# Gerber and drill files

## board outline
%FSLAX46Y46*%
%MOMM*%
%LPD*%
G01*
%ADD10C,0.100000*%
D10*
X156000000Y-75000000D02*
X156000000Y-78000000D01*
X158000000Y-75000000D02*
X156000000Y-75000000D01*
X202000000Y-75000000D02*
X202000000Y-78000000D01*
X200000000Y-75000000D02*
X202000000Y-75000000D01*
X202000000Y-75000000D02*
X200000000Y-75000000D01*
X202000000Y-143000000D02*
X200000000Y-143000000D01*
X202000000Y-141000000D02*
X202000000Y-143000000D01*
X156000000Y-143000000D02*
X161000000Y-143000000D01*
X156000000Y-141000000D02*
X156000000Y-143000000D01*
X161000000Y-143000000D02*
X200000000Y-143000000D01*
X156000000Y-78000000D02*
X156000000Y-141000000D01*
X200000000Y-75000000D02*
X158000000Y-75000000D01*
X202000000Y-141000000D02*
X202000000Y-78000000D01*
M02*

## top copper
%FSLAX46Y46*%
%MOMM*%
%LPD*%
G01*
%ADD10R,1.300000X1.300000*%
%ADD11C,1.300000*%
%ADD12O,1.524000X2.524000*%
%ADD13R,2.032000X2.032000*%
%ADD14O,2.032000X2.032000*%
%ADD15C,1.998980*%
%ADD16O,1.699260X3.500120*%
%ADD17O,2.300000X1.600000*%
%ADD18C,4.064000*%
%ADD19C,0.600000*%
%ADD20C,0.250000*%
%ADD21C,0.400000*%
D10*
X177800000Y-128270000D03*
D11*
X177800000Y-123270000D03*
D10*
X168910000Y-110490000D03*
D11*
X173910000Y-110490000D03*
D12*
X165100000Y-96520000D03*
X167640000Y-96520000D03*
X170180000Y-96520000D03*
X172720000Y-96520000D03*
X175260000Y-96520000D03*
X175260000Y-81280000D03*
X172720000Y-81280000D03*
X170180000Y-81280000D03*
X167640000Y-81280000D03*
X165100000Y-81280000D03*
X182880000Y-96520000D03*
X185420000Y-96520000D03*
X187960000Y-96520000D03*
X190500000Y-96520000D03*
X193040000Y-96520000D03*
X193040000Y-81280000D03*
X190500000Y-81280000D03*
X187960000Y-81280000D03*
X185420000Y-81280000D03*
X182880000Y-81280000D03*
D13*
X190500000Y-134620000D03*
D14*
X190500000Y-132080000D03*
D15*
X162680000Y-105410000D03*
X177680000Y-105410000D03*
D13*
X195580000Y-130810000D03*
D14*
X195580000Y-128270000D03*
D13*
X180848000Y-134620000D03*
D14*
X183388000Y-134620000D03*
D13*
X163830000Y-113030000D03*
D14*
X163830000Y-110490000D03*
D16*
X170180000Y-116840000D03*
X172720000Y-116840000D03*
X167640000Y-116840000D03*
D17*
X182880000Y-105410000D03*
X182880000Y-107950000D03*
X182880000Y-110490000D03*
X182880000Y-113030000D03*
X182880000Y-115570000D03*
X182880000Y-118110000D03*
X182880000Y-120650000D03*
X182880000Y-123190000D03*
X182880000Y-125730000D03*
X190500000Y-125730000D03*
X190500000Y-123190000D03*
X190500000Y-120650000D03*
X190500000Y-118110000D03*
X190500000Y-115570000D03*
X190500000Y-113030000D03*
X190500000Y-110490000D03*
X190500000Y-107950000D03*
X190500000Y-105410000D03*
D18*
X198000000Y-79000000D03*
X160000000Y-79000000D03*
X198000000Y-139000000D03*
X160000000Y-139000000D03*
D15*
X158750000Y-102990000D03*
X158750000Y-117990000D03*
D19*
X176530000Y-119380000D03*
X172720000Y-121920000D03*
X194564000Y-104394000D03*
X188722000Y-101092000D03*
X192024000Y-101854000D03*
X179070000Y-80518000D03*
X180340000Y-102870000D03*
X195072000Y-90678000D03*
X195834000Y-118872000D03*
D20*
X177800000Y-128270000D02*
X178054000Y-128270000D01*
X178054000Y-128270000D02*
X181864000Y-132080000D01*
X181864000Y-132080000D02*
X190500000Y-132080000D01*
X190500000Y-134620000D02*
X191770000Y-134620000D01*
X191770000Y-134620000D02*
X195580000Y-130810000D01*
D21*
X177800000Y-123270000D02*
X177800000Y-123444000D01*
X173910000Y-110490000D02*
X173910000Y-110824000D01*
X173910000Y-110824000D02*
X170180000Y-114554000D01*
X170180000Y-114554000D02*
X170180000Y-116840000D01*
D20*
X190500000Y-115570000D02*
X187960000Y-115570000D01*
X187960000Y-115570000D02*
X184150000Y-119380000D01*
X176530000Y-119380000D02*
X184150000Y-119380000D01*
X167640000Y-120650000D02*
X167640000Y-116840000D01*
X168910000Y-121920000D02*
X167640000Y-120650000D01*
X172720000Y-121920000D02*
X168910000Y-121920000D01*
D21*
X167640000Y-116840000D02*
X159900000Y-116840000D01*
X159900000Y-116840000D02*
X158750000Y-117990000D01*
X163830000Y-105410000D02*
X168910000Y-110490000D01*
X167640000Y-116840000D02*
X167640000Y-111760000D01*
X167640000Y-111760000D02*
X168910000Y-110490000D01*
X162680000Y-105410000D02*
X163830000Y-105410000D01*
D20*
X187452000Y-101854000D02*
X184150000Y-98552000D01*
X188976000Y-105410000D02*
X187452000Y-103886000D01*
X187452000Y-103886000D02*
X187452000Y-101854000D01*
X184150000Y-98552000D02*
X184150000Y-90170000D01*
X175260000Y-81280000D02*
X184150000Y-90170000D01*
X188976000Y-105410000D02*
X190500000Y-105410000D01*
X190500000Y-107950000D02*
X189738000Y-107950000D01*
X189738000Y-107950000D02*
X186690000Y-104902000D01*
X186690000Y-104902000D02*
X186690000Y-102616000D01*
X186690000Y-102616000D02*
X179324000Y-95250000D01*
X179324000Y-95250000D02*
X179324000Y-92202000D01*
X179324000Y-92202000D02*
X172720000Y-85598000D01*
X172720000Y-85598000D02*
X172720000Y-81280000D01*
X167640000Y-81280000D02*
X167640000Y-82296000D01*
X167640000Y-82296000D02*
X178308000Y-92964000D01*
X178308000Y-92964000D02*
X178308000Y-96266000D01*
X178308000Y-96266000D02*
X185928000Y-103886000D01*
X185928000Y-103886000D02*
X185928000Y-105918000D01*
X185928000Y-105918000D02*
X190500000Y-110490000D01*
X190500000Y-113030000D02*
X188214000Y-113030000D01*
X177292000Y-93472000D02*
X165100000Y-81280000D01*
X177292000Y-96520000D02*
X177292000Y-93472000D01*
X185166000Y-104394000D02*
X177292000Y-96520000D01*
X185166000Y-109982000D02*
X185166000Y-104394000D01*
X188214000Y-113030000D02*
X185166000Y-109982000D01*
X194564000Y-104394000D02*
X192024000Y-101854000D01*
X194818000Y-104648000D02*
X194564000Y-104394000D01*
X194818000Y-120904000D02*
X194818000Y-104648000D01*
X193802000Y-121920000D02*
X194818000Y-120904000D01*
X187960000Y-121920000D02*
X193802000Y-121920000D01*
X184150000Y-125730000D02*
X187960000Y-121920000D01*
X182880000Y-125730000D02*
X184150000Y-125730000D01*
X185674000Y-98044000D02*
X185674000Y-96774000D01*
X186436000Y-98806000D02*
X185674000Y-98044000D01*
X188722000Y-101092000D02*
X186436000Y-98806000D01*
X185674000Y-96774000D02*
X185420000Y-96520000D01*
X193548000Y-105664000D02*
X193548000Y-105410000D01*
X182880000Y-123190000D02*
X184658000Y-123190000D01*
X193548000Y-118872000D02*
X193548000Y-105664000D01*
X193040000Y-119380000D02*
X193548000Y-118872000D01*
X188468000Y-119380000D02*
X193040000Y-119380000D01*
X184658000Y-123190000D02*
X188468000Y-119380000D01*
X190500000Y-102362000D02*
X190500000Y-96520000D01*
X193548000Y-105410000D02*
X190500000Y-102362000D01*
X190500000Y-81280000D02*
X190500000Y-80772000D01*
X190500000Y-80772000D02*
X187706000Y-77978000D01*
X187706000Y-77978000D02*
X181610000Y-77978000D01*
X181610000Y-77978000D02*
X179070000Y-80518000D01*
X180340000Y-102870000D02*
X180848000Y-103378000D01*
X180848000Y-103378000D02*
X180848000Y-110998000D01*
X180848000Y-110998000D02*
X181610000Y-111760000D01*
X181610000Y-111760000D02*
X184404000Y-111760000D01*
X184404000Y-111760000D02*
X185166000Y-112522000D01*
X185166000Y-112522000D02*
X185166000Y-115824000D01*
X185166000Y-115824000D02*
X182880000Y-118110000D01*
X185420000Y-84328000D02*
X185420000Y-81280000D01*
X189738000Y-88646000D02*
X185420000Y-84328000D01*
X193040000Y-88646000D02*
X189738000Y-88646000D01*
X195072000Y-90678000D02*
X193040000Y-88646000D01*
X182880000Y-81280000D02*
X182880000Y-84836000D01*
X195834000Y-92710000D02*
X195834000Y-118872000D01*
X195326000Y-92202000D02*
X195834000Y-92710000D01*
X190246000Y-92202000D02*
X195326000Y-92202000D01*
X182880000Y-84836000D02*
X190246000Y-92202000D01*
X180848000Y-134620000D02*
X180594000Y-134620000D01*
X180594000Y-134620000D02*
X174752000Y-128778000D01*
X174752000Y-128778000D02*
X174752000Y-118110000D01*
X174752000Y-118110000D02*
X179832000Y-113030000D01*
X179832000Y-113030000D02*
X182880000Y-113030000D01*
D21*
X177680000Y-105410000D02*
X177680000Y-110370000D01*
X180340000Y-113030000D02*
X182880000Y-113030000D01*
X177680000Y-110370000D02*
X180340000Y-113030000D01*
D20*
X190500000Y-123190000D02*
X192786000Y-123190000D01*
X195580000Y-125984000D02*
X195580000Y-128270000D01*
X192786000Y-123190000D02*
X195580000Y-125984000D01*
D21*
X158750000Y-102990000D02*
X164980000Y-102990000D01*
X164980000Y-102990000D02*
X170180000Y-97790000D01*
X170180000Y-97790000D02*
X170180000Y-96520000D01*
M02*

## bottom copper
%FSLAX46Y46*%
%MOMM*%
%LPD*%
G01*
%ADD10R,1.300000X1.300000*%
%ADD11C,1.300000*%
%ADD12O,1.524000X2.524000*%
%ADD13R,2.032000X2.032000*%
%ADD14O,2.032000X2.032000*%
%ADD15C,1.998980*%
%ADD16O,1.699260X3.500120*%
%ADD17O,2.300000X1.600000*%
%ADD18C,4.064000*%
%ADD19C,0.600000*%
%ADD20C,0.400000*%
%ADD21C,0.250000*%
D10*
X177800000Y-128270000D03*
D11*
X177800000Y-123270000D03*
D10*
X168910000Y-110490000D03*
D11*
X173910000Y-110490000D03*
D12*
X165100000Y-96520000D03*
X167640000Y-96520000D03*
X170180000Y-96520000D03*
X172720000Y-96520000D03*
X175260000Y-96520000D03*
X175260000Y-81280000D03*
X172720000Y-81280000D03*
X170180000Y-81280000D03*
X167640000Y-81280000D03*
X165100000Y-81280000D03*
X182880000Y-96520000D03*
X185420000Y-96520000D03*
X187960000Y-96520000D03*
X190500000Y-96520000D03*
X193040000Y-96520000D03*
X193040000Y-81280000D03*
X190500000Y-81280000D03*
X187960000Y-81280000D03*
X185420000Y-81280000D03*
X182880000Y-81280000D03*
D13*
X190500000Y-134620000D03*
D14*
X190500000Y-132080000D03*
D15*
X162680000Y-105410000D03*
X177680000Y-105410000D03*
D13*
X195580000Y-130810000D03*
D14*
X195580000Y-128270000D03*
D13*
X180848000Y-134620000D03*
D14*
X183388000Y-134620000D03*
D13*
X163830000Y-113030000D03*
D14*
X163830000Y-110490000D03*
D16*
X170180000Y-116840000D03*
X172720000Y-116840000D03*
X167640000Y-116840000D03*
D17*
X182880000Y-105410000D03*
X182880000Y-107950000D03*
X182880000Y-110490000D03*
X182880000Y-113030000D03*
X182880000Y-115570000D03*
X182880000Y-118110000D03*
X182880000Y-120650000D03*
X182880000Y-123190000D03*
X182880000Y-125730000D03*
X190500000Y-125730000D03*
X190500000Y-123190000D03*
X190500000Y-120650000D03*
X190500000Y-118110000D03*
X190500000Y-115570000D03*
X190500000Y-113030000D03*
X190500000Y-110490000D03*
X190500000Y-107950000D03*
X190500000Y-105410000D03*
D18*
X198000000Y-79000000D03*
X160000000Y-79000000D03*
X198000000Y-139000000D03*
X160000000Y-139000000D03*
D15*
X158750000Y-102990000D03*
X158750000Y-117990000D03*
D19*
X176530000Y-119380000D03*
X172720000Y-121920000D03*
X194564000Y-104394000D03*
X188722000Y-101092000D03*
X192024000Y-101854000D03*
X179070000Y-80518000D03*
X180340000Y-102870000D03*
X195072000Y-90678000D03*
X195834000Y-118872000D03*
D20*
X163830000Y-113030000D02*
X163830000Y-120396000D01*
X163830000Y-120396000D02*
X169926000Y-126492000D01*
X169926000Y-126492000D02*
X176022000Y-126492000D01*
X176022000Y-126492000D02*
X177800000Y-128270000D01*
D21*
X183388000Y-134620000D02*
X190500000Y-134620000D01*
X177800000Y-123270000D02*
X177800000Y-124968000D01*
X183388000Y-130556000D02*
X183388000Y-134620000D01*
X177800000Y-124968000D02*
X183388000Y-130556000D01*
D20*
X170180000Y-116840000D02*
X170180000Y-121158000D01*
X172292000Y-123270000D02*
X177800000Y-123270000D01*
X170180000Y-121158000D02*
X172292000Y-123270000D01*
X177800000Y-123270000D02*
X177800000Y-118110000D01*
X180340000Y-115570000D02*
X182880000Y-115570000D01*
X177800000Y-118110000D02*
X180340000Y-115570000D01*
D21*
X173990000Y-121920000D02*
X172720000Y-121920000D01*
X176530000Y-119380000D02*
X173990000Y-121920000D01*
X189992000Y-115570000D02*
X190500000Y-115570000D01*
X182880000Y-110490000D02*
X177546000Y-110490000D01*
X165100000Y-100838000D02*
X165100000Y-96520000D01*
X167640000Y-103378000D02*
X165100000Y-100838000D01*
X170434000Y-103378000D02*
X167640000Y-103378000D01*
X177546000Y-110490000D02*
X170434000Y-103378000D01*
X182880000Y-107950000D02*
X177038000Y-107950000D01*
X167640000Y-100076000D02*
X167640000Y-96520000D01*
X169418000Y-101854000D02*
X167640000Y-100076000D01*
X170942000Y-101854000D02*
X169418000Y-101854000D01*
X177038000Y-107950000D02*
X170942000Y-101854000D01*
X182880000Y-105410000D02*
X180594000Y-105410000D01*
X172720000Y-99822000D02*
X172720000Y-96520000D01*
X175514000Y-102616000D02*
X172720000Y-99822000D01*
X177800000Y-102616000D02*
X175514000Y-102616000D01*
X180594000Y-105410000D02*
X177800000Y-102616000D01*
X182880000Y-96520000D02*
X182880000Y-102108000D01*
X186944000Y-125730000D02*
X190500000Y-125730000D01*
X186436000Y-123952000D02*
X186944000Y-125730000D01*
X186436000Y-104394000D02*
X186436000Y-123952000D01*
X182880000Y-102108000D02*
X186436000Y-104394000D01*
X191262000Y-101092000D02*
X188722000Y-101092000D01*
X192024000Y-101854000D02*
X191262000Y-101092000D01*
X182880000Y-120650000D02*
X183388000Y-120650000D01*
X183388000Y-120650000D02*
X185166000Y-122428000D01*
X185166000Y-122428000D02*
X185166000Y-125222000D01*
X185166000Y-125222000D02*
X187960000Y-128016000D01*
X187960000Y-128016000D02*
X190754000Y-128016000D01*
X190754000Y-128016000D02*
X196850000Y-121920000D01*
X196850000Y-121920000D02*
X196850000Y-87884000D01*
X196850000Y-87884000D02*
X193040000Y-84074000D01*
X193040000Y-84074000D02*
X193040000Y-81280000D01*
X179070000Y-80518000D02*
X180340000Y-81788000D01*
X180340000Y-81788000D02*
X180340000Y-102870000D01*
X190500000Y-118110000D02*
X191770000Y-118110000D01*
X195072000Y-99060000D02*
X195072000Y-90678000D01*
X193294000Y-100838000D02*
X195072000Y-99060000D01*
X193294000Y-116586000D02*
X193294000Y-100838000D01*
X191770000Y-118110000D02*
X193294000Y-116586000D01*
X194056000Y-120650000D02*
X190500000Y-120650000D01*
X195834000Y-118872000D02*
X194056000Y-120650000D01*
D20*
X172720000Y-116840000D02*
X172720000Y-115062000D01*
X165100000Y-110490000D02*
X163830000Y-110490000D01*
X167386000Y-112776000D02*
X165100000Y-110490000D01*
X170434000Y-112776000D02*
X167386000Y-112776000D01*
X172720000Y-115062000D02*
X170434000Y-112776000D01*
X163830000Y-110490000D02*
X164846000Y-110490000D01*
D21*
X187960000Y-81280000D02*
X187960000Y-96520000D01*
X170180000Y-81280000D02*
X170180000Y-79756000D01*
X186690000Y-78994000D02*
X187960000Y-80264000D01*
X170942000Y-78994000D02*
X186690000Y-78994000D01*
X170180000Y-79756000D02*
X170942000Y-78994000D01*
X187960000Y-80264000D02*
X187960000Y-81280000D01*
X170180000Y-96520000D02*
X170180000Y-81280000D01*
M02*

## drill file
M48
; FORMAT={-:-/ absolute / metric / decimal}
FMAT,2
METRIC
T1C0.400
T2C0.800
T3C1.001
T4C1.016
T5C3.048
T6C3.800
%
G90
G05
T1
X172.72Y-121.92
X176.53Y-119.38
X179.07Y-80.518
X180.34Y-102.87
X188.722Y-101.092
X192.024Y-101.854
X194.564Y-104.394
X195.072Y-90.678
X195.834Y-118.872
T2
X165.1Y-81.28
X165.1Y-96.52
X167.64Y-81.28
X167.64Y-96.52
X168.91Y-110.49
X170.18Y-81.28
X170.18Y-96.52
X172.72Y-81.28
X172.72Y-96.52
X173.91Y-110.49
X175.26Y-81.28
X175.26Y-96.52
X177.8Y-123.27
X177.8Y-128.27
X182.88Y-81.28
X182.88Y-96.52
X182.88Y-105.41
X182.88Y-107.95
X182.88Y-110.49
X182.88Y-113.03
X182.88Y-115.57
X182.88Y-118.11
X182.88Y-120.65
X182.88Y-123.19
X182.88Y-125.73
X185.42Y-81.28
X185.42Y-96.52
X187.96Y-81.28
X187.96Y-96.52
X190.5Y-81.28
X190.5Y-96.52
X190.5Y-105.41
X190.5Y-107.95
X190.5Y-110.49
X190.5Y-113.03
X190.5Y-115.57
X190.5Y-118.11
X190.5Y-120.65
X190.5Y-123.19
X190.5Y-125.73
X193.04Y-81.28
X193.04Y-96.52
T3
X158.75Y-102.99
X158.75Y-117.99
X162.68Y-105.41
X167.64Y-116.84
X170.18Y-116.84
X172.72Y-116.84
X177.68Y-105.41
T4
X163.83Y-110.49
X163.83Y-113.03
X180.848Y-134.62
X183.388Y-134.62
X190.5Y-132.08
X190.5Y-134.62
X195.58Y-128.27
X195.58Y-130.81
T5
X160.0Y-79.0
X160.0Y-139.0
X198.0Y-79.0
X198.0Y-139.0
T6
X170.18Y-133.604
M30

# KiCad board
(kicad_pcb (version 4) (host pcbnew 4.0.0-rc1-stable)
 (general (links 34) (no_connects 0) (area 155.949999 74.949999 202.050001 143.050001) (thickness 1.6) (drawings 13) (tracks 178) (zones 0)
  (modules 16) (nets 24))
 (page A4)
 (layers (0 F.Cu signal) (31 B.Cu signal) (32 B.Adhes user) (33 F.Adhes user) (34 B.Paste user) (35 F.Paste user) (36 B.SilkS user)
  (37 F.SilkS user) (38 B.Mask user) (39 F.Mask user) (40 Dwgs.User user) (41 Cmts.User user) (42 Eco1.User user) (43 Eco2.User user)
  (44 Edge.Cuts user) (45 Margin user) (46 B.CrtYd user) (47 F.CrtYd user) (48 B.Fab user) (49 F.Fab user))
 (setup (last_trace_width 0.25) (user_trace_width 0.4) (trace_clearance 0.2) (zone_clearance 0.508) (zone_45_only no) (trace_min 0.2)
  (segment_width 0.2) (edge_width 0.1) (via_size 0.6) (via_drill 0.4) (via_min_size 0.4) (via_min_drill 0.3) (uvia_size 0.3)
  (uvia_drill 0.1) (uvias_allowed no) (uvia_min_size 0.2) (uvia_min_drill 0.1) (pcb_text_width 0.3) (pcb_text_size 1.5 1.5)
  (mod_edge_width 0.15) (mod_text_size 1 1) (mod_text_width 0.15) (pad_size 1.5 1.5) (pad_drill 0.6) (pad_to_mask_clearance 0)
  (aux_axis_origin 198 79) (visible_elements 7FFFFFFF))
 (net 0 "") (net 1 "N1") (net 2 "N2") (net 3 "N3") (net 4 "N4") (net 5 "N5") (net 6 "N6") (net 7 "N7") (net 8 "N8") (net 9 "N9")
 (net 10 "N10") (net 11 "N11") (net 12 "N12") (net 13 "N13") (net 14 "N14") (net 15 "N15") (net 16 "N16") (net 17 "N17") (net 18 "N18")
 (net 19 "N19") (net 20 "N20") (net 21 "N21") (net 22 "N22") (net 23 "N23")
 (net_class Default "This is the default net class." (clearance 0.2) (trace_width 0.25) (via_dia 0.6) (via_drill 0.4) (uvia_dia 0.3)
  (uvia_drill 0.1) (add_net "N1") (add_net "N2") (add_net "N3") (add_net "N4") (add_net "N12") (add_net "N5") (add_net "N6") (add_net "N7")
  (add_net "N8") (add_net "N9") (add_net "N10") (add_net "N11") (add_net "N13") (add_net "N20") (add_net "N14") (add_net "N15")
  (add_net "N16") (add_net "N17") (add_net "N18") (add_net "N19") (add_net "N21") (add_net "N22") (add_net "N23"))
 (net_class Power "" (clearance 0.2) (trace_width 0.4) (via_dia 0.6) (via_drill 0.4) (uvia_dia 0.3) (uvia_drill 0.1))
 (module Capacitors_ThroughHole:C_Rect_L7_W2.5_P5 (layer F.Cu) (at 177.8 128.27 90)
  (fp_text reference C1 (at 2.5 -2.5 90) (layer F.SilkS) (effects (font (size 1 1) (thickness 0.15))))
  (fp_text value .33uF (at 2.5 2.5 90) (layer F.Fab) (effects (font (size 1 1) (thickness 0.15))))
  (pad 1 thru_hole rect (at 0 0 90) (size 1.3 1.3) (drill 0.8) (layers *.Cu *.Mask F.SilkS) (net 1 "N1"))
  (pad 2 thru_hole circle (at 5 0 90) (size 1.3 1.3) (drill 0.8) (layers *.Cu *.Mask F.SilkS) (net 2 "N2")))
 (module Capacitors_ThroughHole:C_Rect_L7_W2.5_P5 (layer F.Cu) (at 168.91 110.49)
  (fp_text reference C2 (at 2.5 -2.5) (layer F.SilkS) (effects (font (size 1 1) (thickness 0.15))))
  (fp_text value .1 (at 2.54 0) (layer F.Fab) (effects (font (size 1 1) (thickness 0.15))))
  (pad 1 thru_hole rect (at 0 0) (size 1.3 1.3) (drill 0.8) (layers *.Cu *.Mask F.SilkS) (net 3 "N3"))
  (pad 2 thru_hole circle (at 5 0) (size 1.3 1.3) (drill 0.8) (layers *.Cu *.Mask F.SilkS) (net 2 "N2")))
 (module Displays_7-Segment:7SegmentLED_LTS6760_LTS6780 (layer F.Cu) (at 170.18 88.9)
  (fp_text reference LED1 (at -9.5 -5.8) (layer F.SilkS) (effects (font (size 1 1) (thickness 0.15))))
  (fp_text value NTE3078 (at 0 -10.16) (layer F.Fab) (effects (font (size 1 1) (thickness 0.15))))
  (pad 1 thru_hole oval (at -5.08 7.62) (size 1.524 2.524) (drill 0.8) (layers *.Cu *.Mask F.SilkS) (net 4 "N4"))
  (pad 2 thru_hole oval (at -2.54 7.62) (size 1.524 2.524) (drill 0.8) (layers *.Cu *.Mask F.SilkS) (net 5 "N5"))
  (pad 3 thru_hole oval (at 0 7.62) (size 1.524 2.524) (drill 0.8) (layers *.Cu *.Mask F.SilkS) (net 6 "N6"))
  (pad 4 thru_hole oval (at 2.54 7.62) (size 1.524 2.524) (drill 0.8) (layers *.Cu *.Mask F.SilkS) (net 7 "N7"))
  (pad 5 thru_hole oval (at 5.08 7.62) (size 1.524 2.524) (drill 0.8) (layers *.Cu *.Mask F.SilkS) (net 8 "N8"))
  (pad 6 thru_hole oval (at 5.08 -7.62) (size 1.524 2.524) (drill 0.8) (layers *.Cu *.Mask F.SilkS) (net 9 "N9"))
  (pad 7 thru_hole oval (at 2.54 -7.62) (size 1.524 2.524) (drill 0.8) (layers *.Cu *.Mask F.SilkS) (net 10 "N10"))
  (pad 8 thru_hole oval (at 0 -7.62) (size 1.524 2.524) (drill 0.8) (layers *.Cu *.Mask F.SilkS) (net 6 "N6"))
  (pad 9 thru_hole oval (at -2.54 -7.62) (size 1.524 2.524) (drill 0.8) (layers *.Cu *.Mask F.SilkS) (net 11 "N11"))
  (pad 10 thru_hole oval (at -5.08 -7.62) (size 1.524 2.524) (drill 0.8) (layers *.Cu *.Mask F.SilkS) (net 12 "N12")))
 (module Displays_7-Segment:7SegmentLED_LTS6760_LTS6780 (layer F.Cu) (at 187.96 88.9)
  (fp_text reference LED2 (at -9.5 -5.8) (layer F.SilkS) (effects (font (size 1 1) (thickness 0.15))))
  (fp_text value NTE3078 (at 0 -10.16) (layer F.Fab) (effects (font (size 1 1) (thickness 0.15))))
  (pad 1 thru_hole oval (at -5.08 7.62) (size 1.524 2.524) (drill 0.8) (layers *.Cu *.Mask F.SilkS) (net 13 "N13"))
  (pad 2 thru_hole oval (at -2.54 7.62) (size 1.524 2.524) (drill 0.8) (layers *.Cu *.Mask F.SilkS) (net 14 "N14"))
  (pad 3 thru_hole oval (at 0 7.62) (size 1.524 2.524) (drill 0.8) (layers *.Cu *.Mask F.SilkS) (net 6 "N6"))
  (pad 4 thru_hole oval (at 2.54 7.62) (size 1.524 2.524) (drill 0.8) (layers *.Cu *.Mask F.SilkS) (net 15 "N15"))
  (pad 5 thru_hole oval (at 5.08 7.62) (size 1.524 2.524) (drill 0.8) (layers *.Cu *.Mask F.SilkS) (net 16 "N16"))
  (pad 6 thru_hole oval (at 5.08 -7.62) (size 1.524 2.524) (drill 0.8) (layers *.Cu *.Mask F.SilkS) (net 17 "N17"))
  (pad 7 thru_hole oval (at 2.54 -7.62) (size 1.524 2.524) (drill 0.8) (layers *.Cu *.Mask F.SilkS) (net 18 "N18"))
  (pad 8 thru_hole oval (at 0 -7.62) (size 1.524 2.524) (drill 0.8) (layers *.Cu *.Mask F.SilkS) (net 6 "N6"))
  (pad 9 thru_hole oval (at -2.54 -7.62) (size 1.524 2.524) (drill 0.8) (layers *.Cu *.Mask F.SilkS) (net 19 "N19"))
  (pad 10 thru_hole oval (at -5.08 -7.62) (size 1.524 2.524) (drill 0.8) (layers *.Cu *.Mask F.SilkS) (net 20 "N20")))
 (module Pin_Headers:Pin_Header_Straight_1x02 (layer F.Cu) (at 190.5 134.62 180)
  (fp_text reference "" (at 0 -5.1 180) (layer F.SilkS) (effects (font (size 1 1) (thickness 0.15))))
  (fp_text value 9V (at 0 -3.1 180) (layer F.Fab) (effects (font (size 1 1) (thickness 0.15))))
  (pad 1 thru_hole rect (at 0 0 180) (size 2.032 2.032) (drill 1.016) (layers *.Cu *.Mask F.SilkS) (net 2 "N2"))
  (pad 2 thru_hole oval (at 0 2.54 180) (size 2.032 2.032) (drill 1.016) (layers *.Cu *.Mask F.SilkS) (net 1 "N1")))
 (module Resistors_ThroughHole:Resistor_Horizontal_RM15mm (layer F.Cu) (at 170.18 105.41)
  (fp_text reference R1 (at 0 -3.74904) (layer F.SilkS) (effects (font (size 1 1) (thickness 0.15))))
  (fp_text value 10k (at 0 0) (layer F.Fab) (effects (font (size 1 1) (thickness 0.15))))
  (pad 1 thru_hole circle (at -7.5 0) (size 1.99898 1.99898) (drill 1.00076) (layers *.Cu *.SilkS *.Mask) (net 3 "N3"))
  (pad 2 thru_hole circle (at 7.5 0) (size 1.99898 1.99898) (drill 1.00076) (layers *.Cu *.SilkS *.Mask) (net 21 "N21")))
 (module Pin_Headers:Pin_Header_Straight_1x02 (layer F.Cu) (at 195.58 130.81 180)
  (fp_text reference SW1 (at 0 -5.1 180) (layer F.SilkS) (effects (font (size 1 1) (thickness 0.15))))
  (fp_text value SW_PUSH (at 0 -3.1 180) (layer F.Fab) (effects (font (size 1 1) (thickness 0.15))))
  (pad 1 thru_hole rect (at 0 0 180) (size 2.032 2.032) (drill 1.016) (layers *.Cu *.Mask F.SilkS) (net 2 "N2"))
  (pad 2 thru_hole oval (at 0 2.54 180) (size 2.032 2.032) (drill 1.016) (layers *.Cu *.Mask F.SilkS) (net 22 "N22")))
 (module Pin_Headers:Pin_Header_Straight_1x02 (layer F.Cu) (at 180.848 134.62 90)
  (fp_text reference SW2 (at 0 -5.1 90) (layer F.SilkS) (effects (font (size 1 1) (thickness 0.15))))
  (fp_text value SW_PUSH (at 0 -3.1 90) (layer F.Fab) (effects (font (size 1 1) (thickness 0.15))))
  (pad 1 thru_hole rect (at 0 0 90) (size 2.032 2.032) (drill 1.016) (layers *.Cu *.Mask F.SilkS) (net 21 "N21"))
  (pad 2 thru_hole oval (at 0 2.54 90) (size 2.032 2.032) (drill 1.016) (layers *.Cu *.Mask F.SilkS) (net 2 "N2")))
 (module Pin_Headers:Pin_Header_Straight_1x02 (layer F.Cu) (at 163.83 113.03 180)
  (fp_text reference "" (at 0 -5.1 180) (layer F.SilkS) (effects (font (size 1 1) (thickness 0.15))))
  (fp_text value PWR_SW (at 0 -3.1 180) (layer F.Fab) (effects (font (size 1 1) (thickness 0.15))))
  (pad 1 thru_hole rect (at 0 0 180) (size 2.032 2.032) (drill 1.016) (layers *.Cu *.Mask F.SilkS) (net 1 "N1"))
  (pad 2 thru_hole oval (at 0 2.54 180) (size 2.032 2.032) (drill 1.016) (layers *.Cu *.Mask F.SilkS) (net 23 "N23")))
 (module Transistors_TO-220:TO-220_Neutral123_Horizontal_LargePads (layer F.Cu) (at 170.18 116.84 180)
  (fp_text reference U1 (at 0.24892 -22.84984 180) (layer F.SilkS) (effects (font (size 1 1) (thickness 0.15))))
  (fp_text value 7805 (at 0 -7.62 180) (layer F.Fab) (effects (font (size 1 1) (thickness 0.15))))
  (pad 2 thru_hole oval (at 0 0 270) (size 3.50012 1.69926) (drill 1.00076) (layers *.Cu *.Mask F.SilkS) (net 2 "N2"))
  (pad 1 thru_hole oval (at -2.54 0 270) (size 3.50012 1.69926) (drill 1.00076) (layers *.Cu *.Mask F.SilkS) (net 23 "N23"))
  (pad 3 thru_hole oval (at 2.54 0 270) (size 3.50012 1.69926) (drill 1.00076) (layers *.Cu *.Mask F.SilkS) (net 3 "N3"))
  (pad "" np_thru_hole circle (at 0 -16.764 270) (size 3.79984 3.79984) (drill 3.79984) (layers *.Cu *.Mask F.SilkS)))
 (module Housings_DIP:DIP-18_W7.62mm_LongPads (layer F.Cu) (at 182.88 105.41)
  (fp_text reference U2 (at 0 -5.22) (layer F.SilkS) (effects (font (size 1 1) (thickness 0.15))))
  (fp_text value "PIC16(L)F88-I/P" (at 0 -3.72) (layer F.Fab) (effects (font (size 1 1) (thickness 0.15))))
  (pad 1 thru_hole oval (at 0 0) (size 2.3 1.6) (drill 0.8) (layers *.Cu *.Mask F.SilkS) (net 7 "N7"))
  (pad 2 thru_hole oval (at 0 2.54) (size 2.3 1.6) (drill 0.8) (layers *.Cu *.Mask F.SilkS) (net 5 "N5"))
  (pad 3 thru_hole oval (at 0 5.08) (size 2.3 1.6) (drill 0.8) (layers *.Cu *.Mask F.SilkS) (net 4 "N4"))
  (pad 4 thru_hole oval (at 0 7.62) (size 2.3 1.6) (drill 0.8) (layers *.Cu *.Mask F.SilkS) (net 21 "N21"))
  (pad 5 thru_hole oval (at 0 10.16) (size 2.3 1.6) (drill 0.8) (layers *.Cu *.Mask F.SilkS) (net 2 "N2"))
  (pad 6 thru_hole oval (at 0 12.7) (size 2.3 1.6) (drill 0.8) (layers *.Cu *.Mask F.SilkS) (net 18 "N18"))
  (pad 7 thru_hole oval (at 0 15.24) (size 2.3 1.6) (drill 0.8) (layers *.Cu *.Mask F.SilkS) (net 17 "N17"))
  (pad 8 thru_hole oval (at 0 17.78) (size 2.3 1.6) (drill 0.8) (layers *.Cu *.Mask F.SilkS) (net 15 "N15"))
  (pad 9 thru_hole oval (at 0 20.32) (size 2.3 1.6) (drill 0.8) (layers *.Cu *.Mask F.SilkS) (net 14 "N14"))
  (pad 10 thru_hole oval (at 7.62 20.32) (size 2.3 1.6) (drill 0.8) (layers *.Cu *.Mask F.SilkS) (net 13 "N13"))
  (pad 11 thru_hole oval (at 7.62 17.78) (size 2.3 1.6) (drill 0.8) (layers *.Cu *.Mask F.SilkS) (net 22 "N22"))
  (pad 12 thru_hole oval (at 7.62 15.24) (size 2.3 1.6) (drill 0.8) (layers *.Cu *.Mask F.SilkS) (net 20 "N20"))
  (pad 13 thru_hole oval (at 7.62 12.7) (size 2.3 1.6) (drill 0.8) (layers *.Cu *.Mask F.SilkS) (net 19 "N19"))
  (pad 14 thru_hole oval (at 7.62 10.16) (size 2.3 1.6) (drill 0.8) (layers *.Cu *.Mask F.SilkS) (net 3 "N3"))
  (pad 15 thru_hole oval (at 7.62 7.62) (size 2.3 1.6) (drill 0.8) (layers *.Cu *.Mask F.SilkS) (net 12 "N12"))
  (pad 16 thru_hole oval (at 7.62 5.08) (size 2.3 1.6) (drill 0.8) (layers *.Cu *.Mask F.SilkS) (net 11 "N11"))
  (pad 17 thru_hole oval (at 7.62 2.54) (size 2.3 1.6) (drill 0.8) (layers *.Cu *.Mask F.SilkS) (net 10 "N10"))
  (pad 18 thru_hole oval (at 7.62 0) (size 2.3 1.6) (drill 0.8) (layers *.Cu *.Mask F.SilkS) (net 9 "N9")))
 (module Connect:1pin (layer F.Cu) (at 198 79)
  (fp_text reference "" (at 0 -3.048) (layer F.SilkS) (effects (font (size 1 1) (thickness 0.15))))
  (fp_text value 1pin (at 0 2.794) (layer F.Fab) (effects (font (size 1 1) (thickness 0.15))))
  (pad 1 thru_hole circle (at 0 0) (size 4.064 4.064) (drill 3.048) (layers *.Cu *.Mask F.SilkS)))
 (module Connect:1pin (layer F.Cu) (at 160 79)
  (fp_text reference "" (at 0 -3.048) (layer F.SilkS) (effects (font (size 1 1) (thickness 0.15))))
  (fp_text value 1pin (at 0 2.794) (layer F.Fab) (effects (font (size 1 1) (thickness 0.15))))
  (pad 1 thru_hole circle (at 0 0) (size 4.064 4.064) (drill 3.048) (layers *.Cu *.Mask F.SilkS)))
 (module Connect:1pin (layer F.Cu) (at 198 139)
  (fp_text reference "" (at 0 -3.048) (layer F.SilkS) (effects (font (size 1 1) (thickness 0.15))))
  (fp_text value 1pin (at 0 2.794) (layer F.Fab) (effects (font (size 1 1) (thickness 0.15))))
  (pad 1 thru_hole circle (at 0 0) (size 4.064 4.064) (drill 3.048) (layers *.Cu *.Mask F.SilkS)))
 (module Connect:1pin (layer F.Cu) (at 160 139)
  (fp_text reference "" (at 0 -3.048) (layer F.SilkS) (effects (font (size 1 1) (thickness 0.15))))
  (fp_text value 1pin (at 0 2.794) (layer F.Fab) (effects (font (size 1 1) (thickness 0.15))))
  (pad 1 thru_hole circle (at 0 0) (size 4.064 4.064) (drill 3.048) (layers *.Cu *.Mask F.SilkS)))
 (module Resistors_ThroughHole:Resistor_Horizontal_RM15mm (layer F.Cu) (at 158.75 110.49 270)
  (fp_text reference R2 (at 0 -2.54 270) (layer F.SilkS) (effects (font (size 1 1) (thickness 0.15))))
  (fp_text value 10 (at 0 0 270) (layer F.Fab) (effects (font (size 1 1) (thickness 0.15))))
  (pad 1 thru_hole circle (at -7.5 0 270) (size 1.99898 1.99898) (drill 1.00076) (layers *.Cu *.SilkS *.Mask) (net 6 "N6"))
  (pad 2 thru_hole circle (at 7.5 0 270) (size 1.99898 1.99898) (drill 1.00076) (layers *.Cu *.SilkS *.Mask) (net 3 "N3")))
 (gr_line (start 156 75) (end 156 78) (angle 90) (layer Edge.Cuts) (width 0.1))
 (gr_line (start 158 75) (end 156 75) (angle 90) (layer Edge.Cuts) (width 0.1))
 (gr_line (start 202 75) (end 202 78) (angle 90) (layer Edge.Cuts) (width 0.1))
 (gr_line (start 200 75) (end 202 75) (angle 90) (layer Edge.Cuts) (width 0.1))
 (gr_line (start 202 75) (end 200 75) (angle 90) (layer Edge.Cuts) (width 0.1))
 (gr_line (start 202 143) (end 200 143) (angle 90) (layer Edge.Cuts) (width 0.1))
 (gr_line (start 202 141) (end 202 143) (angle 90) (layer Edge.Cuts) (width 0.1))
 (gr_line (start 156 143) (end 161 143) (angle 90) (layer Edge.Cuts) (width 0.1))
 (gr_line (start 156 141) (end 156 143) (angle 90) (layer Edge.Cuts) (width 0.1))
 (gr_line (start 161 143) (end 200 143) (angle 90) (layer Edge.Cuts) (width 0.1))
 (gr_line (start 156 78) (end 156 141) (angle 90) (layer Edge.Cuts) (width 0.1))
 (gr_line (start 200 75) (end 158 75) (angle 90) (layer Edge.Cuts) (width 0.1))
 (gr_line (start 202 141) (end 202 78) (angle 90) (layer Edge.Cuts) (width 0.1))
 (segment (start 177.8 128.27) (end 178.054 128.27) (width 0.25) (layer F.Cu) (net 1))
 (segment (start 178.054 128.27) (end 181.864 132.08) (width 0.25) (layer F.Cu) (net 1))
 (segment (start 181.864 132.08) (end 190.5 132.08) (width 0.25) (layer F.Cu) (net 1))
 (segment (start 163.83 113.03) (end 163.83 120.396) (width 0.4) (layer B.Cu) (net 1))
 (segment (start 163.83 120.396) (end 169.926 126.492) (width 0.4) (layer B.Cu) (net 1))
 (segment (start 169.926 126.492) (end 176.022 126.492) (width 0.4) (layer B.Cu) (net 1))
 (segment (start 176.022 126.492) (end 177.8 128.27) (width 0.4) (layer B.Cu) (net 1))
 (segment (start 190.5 134.62) (end 191.77 134.62) (width 0.25) (layer F.Cu) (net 2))
 (segment (start 191.77 134.62) (end 195.58 130.81) (width 0.25) (layer F.Cu) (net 2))
 (segment (start 183.388 134.62) (end 190.5 134.62) (width 0.25) (layer B.Cu) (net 2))
 (segment (start 177.8 123.27) (end 177.8 124.968) (width 0.25) (layer B.Cu) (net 2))
 (segment (start 183.388 130.556) (end 183.388 134.62) (width 0.25) (layer B.Cu) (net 2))
 (segment (start 177.8 124.968) (end 183.388 130.556) (width 0.25) (layer B.Cu) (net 2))
 (segment (start 177.8 123.27) (end 177.8 123.444) (width 0.4) (layer F.Cu) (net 2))
 (segment (start 170.18 116.84) (end 170.18 121.158) (width 0.4) (layer B.Cu) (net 2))
 (segment (start 172.292 123.27) (end 177.8 123.27) (width 0.4) (layer B.Cu) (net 2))
 (segment (start 170.18 121.158) (end 172.292 123.27) (width 0.4) (layer B.Cu) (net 2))
 (segment (start 177.8 123.27) (end 177.8 118.11) (width 0.4) (layer B.Cu) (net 2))
 (segment (start 180.34 115.57) (end 182.88 115.57) (width 0.4) (layer B.Cu) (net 2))
 (segment (start 177.8 118.11) (end 180.34 115.57) (width 0.4) (layer B.Cu) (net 2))
 (segment (start 173.91 110.49) (end 173.91 110.824) (width 0.4) (layer F.Cu) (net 2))
 (segment (start 173.91 110.824) (end 170.18 114.554) (width 0.4) (layer F.Cu) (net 2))
 (segment (start 170.18 114.554) (end 170.18 116.84) (width 0.4) (layer F.Cu) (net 2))
 (via (at 176.53 119.38) (size 0.6) (drill 0.4) (layers F.Cu B.Cu) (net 3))
 (segment (start 190.5 115.57) (end 187.96 115.57) (width 0.25) (layer F.Cu) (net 3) (status 400000))
 (segment (start 187.96 115.57) (end 184.15 119.38) (width 0.25) (layer F.Cu) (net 3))
 (segment (start 176.53 119.38) (end 184.15 119.38) (width 0.25) (layer F.Cu) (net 3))
 (segment (start 167.64 120.65) (end 167.64 116.84) (width 0.25) (layer F.Cu) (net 3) (status 800000))
 (segment (start 168.91 121.92) (end 167.64 120.65) (width 0.25) (layer F.Cu) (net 3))
 (segment (start 172.72 121.92) (end 168.91 121.92) (width 0.25) (layer F.Cu) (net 3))
 (via (at 172.72 121.92) (size 0.6) (drill 0.4) (layers F.Cu B.Cu) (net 3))
 (segment (start 173.99 121.92) (end 172.72 121.92) (width 0.25) (layer B.Cu) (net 3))
 (segment (start 176.53 119.38) (end 173.99 121.92) (width 0.25) (layer B.Cu) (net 3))
 (segment (start 167.64 116.84) (end 159.9 116.84) (width 0.4) (layer F.Cu) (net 3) (status 400000))
 (segment (start 159.9 116.84) (end 158.75 117.99) (width 0.4) (layer F.Cu) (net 3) (status 800000))
 (segment (start 189.992 115.57) (end 190.5 115.57) (width 0.25) (layer B.Cu) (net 3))
 (segment (start 163.83 105.41) (end 168.91 110.49) (width 0.4) (layer F.Cu) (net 3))
 (segment (start 167.64 116.84) (end 167.64 111.76) (width 0.4) (layer F.Cu) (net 3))
 (segment (start 167.64 111.76) (end 168.91 110.49) (width 0.4) (layer F.Cu) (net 3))
 (segment (start 162.68 105.41) (end 163.83 105.41) (width 0.4) (layer F.Cu) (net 3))
 (segment (start 182.88 110.49) (end 177.546 110.49) (width 0.25) (layer B.Cu) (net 4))
 (segment (start 165.1 100.838) (end 165.1 96.52) (width 0.25) (layer B.Cu) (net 4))
 (segment (start 167.64 103.378) (end 165.1 100.838) (width 0.25) (layer B.Cu) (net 4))
 (segment (start 170.434 103.378) (end 167.64 103.378) (width 0.25) (layer B.Cu) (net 4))
 (segment (start 177.546 110.49) (end 170.434 103.378) (width 0.25) (layer B.Cu) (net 4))
 (segment (start 182.88 107.95) (end 177.038 107.95) (width 0.25) (layer B.Cu) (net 5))
 (segment (start 167.64 100.076) (end 167.64 96.52) (width 0.25) (layer B.Cu) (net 5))
 (segment (start 169.418 101.854) (end 167.64 100.076) (width 0.25) (layer B.Cu) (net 5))
 (segment (start 170.942 101.854) (end 169.418 101.854) (width 0.25) (layer B.Cu) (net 5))
 (segment (start 177.038 107.95) (end 170.942 101.854) (width 0.25) (layer B.Cu) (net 5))
 (segment (start 182.88 105.41) (end 180.594 105.41) (width 0.25) (layer B.Cu) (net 7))
 (segment (start 172.72 99.822) (end 172.72 96.52) (width 0.25) (layer B.Cu) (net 7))
 (segment (start 175.514 102.616) (end 172.72 99.822) (width 0.25) (layer B.Cu) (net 7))
 (segment (start 177.8 102.616) (end 175.514 102.616) (width 0.25) (layer B.Cu) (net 7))
 (segment (start 180.594 105.41) (end 177.8 102.616) (width 0.25) (layer B.Cu) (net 7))
 (segment (start 187.452 101.854) (end 184.15 98.552) (width 0.25) (layer F.Cu) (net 9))
 (segment (start 188.976 105.41) (end 187.452 103.886) (width 0.25) (layer F.Cu) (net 9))
 (segment (start 187.452 103.886) (end 187.452 101.854) (width 0.25) (layer F.Cu) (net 9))
 (segment (start 184.15 98.552) (end 184.15 90.17) (width 0.25) (layer F.Cu) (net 9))
 (segment (start 175.26 81.28) (end 184.15 90.17) (width 0.25) (layer F.Cu) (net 9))
 (segment (start 188.976 105.41) (end 190.5 105.41) (width 0.25) (layer F.Cu) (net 9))
 (segment (start 190.5 107.95) (end 189.738 107.95) (width 0.25) (layer F.Cu) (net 10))
 (segment (start 189.738 107.95) (end 186.69 104.902) (width 0.25) (layer F.Cu) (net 10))
 (segment (start 186.69 104.902) (end 186.69 102.616) (width 0.25) (layer F.Cu) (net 10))
 (segment (start 186.69 102.616) (end 179.324 95.25) (width 0.25) (layer F.Cu) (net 10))
 (segment (start 179.324 95.25) (end 179.324 92.202) (width 0.25) (layer F.Cu) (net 10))
 (segment (start 179.324 92.202) (end 172.72 85.598) (width 0.25) (layer F.Cu) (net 10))
 (segment (start 172.72 85.598) (end 172.72 81.28) (width 0.25) (layer F.Cu) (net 10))
 (segment (start 167.64 81.28) (end 167.64 82.296) (width 0.25) (layer F.Cu) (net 11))
 (segment (start 167.64 82.296) (end 178.308 92.964) (width 0.25) (layer F.Cu) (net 11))
 (segment (start 178.308 92.964) (end 178.308 96.266) (width 0.25) (layer F.Cu) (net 11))
 (segment (start 178.308 96.266) (end 185.928 103.886) (width 0.25) (layer F.Cu) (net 11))
 (segment (start 185.928 103.886) (end 185.928 105.918) (width 0.25) (layer F.Cu) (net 11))
 (segment (start 185.928 105.918) (end 190.5 110.49) (width 0.25) (layer F.Cu) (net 11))
 (segment (start 190.5 113.03) (end 188.214 113.03) (width 0.25) (layer F.Cu) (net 12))
 (segment (start 177.292 93.472) (end 165.1 81.28) (width 0.25) (layer F.Cu) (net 12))
 (segment (start 177.292 96.52) (end 177.292 93.472) (width 0.25) (layer F.Cu) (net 12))
 (segment (start 185.166 104.394) (end 177.292 96.52) (width 0.25) (layer F.Cu) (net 12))
 (segment (start 185.166 109.982) (end 185.166 104.394) (width 0.25) (layer F.Cu) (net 12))
 (segment (start 188.214 113.03) (end 185.166 109.982) (width 0.25) (layer F.Cu) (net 12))
 (segment (start 182.88 96.52) (end 182.88 102.108) (width 0.25) (layer B.Cu) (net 13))
 (segment (start 186.944 125.73) (end 190.5 125.73) (width 0.25) (layer B.Cu) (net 13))
 (segment (start 186.436 123.952) (end 186.944 125.73) (width 0.25) (layer B.Cu) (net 13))
 (segment (start 186.436 104.394) (end 186.436 123.952) (width 0.25) (layer B.Cu) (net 13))
 (segment (start 182.88 102.108) (end 186.436 104.394) (width 0.25) (layer B.Cu) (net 13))
 (segment (start 194.564 104.394) (end 192.024 101.854) (width 0.25) (layer F.Cu) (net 14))
 (via (at 194.564 104.394) (size 0.6) (drill 0.4) (layers F.Cu B.Cu) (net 14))
 (segment (start 194.818 104.648) (end 194.564 104.394) (width 0.25) (layer F.Cu) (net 14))
 (segment (start 194.818 120.904) (end 194.818 104.648) (width 0.25) (layer F.Cu) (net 14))
 (segment (start 193.802 121.92) (end 194.818 120.904) (width 0.25) (layer F.Cu) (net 14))
 (segment (start 187.96 121.92) (end 193.802 121.92) (width 0.25) (layer F.Cu) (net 14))
 (segment (start 184.15 125.73) (end 187.96 121.92) (width 0.25) (layer F.Cu) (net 14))
 (segment (start 182.88 125.73) (end 184.15 125.73) (width 0.25) (layer F.Cu) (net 14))
 (segment (start 185.674 98.044) (end 185.674 96.774) (width 0.25) (layer F.Cu) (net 14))
 (segment (start 186.436 98.806) (end 185.674 98.044) (width 0.25) (layer F.Cu) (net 14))
 (segment (start 188.722 101.092) (end 186.436 98.806) (width 0.25) (layer F.Cu) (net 14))
 (via (at 188.722 101.092) (size 0.6) (drill 0.4) (layers F.Cu B.Cu) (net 14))
 (segment (start 191.262 101.092) (end 188.722 101.092) (width 0.25) (layer B.Cu) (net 14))
 (segment (start 192.024 101.854) (end 191.262 101.092) (width 0.25) (layer B.Cu) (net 14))
 (via (at 192.024 101.854) (size 0.6) (drill 0.4) (layers F.Cu B.Cu) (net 14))
 (segment (start 185.674 96.774) (end 185.42 96.52) (width 0.25) (layer F.Cu) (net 14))
 (segment (start 193.548 105.664) (end 193.548 105.41) (width 0.25) (layer F.Cu) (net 15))
 (segment (start 182.88 123.19) (end 184.658 123.19) (width 0.25) (layer F.Cu) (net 15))
 (segment (start 193.548 118.872) (end 193.548 105.664) (width 0.25) (layer F.Cu) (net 15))
 (segment (start 193.04 119.38) (end 193.548 118.872) (width 0.25) (layer F.Cu) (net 15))
 (segment (start 188.468 119.38) (end 193.04 119.38) (width 0.25) (layer F.Cu) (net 15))
 (segment (start 184.658 123.19) (end 188.468 119.38) (width 0.25) (layer F.Cu) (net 15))
 (segment (start 190.5 102.362) (end 190.5 96.52) (width 0.25) (layer F.Cu) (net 15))
 (segment (start 193.548 105.41) (end 190.5 102.362) (width 0.25) (layer F.Cu) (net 15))
 (segment (start 182.88 120.65) (end 183.388 120.65) (width 0.25) (layer B.Cu) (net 17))
 (segment (start 183.388 120.65) (end 185.166 122.428) (width 0.25) (layer B.Cu) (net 17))
 (segment (start 185.166 122.428) (end 185.166 125.222) (width 0.25) (layer B.Cu) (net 17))
 (segment (start 185.166 125.222) (end 187.96 128.016) (width 0.25) (layer B.Cu) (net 17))
 (segment (start 187.96 128.016) (end 190.754 128.016) (width 0.25) (layer B.Cu) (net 17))
 (segment (start 190.754 128.016) (end 196.85 121.92) (width 0.25) (layer B.Cu) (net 17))
 (segment (start 196.85 121.92) (end 196.85 87.884) (width 0.25) (layer B.Cu) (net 17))
 (segment (start 196.85 87.884) (end 193.04 84.074) (width 0.25) (layer B.Cu) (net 17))
 (segment (start 193.04 84.074) (end 193.04 81.28) (width 0.25) (layer B.Cu) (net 17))
 (segment (start 190.5 81.28) (end 190.5 80.772) (width 0.25) (layer F.Cu) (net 18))
 (segment (start 190.5 80.772) (end 187.706 77.978) (width 0.25) (layer F.Cu) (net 18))
 (segment (start 187.706 77.978) (end 181.61 77.978) (width 0.25) (layer F.Cu) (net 18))
 (segment (start 181.61 77.978) (end 179.07 80.518) (width 0.25) (layer F.Cu) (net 18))
 (via (at 179.07 80.518) (size 0.6) (drill 0.4) (layers F.Cu B.Cu) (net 18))
 (segment (start 179.07 80.518) (end 180.34 81.788) (width 0.25) (layer B.Cu) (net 18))
 (segment (start 180.34 81.788) (end 180.34 102.87) (width 0.25) (layer B.Cu) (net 18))
 (via (at 180.34 102.87) (size 0.6) (drill 0.4) (layers F.Cu B.Cu) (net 18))
 (segment (start 180.34 102.87) (end 180.848 103.378) (width 0.25) (layer F.Cu) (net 18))
 (segment (start 180.848 103.378) (end 180.848 110.998) (width 0.25) (layer F.Cu) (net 18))
 (segment (start 180.848 110.998) (end 181.61 111.76) (width 0.25) (layer F.Cu) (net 18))
 (segment (start 181.61 111.76) (end 184.404 111.76) (width 0.25) (layer F.Cu) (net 18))
 (segment (start 184.404 111.76) (end 185.166 112.522) (width 0.25) (layer F.Cu) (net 18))
 (segment (start 185.166 112.522) (end 185.166 115.824) (width 0.25) (layer F.Cu) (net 18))
 (segment (start 185.166 115.824) (end 182.88 118.11) (width 0.25) (layer F.Cu) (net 18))
 (segment (start 190.5 118.11) (end 191.77 118.11) (width 0.25) (layer B.Cu) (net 19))
 (segment (start 185.42 84.328) (end 185.42 81.28) (width 0.25) (layer F.Cu) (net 19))
 (segment (start 189.738 88.646) (end 185.42 84.328) (width 0.25) (layer F.Cu) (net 19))
 (segment (start 193.04 88.646) (end 189.738 88.646) (width 0.25) (layer F.Cu) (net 19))
 (segment (start 195.072 90.678) (end 193.04 88.646) (width 0.25) (layer F.Cu) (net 19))
 (via (at 195.072 90.678) (size 0.6) (drill 0.4) (layers F.Cu B.Cu) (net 19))
 (segment (start 195.072 99.06) (end 195.072 90.678) (width 0.25) (layer B.Cu) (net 19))
 (segment (start 193.294 100.838) (end 195.072 99.06) (width 0.25) (layer B.Cu) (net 19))
 (segment (start 193.294 116.586) (end 193.294 100.838) (width 0.25) (layer B.Cu) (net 19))
 (segment (start 191.77 118.11) (end 193.294 116.586) (width 0.25) (layer B.Cu) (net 19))
 (segment (start 182.88 81.28) (end 182.88 84.836) (width 0.25) (layer F.Cu) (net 20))
 (segment (start 194.056 120.65) (end 190.5 120.65) (width 0.25) (layer B.Cu) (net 20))
 (segment (start 195.834 118.872) (end 194.056 120.65) (width 0.25) (layer B.Cu) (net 20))
 (via (at 195.834 118.872) (size 0.6) (drill 0.4) (layers F.Cu B.Cu) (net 20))
 (segment (start 195.834 92.71) (end 195.834 118.872) (width 0.25) (layer F.Cu) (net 20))
 (segment (start 195.326 92.202) (end 195.834 92.71) (width 0.25) (layer F.Cu) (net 20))
 (segment (start 190.246 92.202) (end 195.326 92.202) (width 0.25) (layer F.Cu) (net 20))
 (segment (start 182.88 84.836) (end 190.246 92.202) (width 0.25) (layer F.Cu) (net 20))
 (segment (start 180.848 134.62) (end 180.594 134.62) (width 0.25) (layer F.Cu) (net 21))
 (segment (start 180.594 134.62) (end 174.752 128.778) (width 0.25) (layer F.Cu) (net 21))
 (segment (start 174.752 128.778) (end 174.752 118.11) (width 0.25) (layer F.Cu) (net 21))
 (segment (start 174.752 118.11) (end 179.832 113.03) (width 0.25) (layer F.Cu) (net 21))
 (segment (start 179.832 113.03) (end 182.88 113.03) (width 0.25) (layer F.Cu) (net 21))
 (segment (start 177.68 105.41) (end 177.68 110.37) (width 0.4) (layer F.Cu) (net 21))
 (segment (start 180.34 113.03) (end 182.88 113.03) (width 0.4) (layer F.Cu) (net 21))
 (segment (start 177.68 110.37) (end 180.34 113.03) (width 0.4) (layer F.Cu) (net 21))
 (segment (start 190.5 123.19) (end 192.786 123.19) (width 0.25) (layer F.Cu) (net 22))
 (segment (start 195.58 125.984) (end 195.58 128.27) (width 0.25) (layer F.Cu) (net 22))
 (segment (start 192.786 123.19) (end 195.58 125.984) (width 0.25) (layer F.Cu) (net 22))
 (segment (start 172.72 116.84) (end 172.72 115.062) (width 0.4) (layer B.Cu) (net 23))
 (segment (start 165.1 110.49) (end 163.83 110.49) (width 0.4) (layer B.Cu) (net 23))
 (segment (start 167.386 112.776) (end 165.1 110.49) (width 0.4) (layer B.Cu) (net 23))
 (segment (start 170.434 112.776) (end 167.386 112.776) (width 0.4) (layer B.Cu) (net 23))
 (segment (start 172.72 115.062) (end 170.434 112.776) (width 0.4) (layer B.Cu) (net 23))
 (segment (start 163.83 110.49) (end 164.846 110.49) (width 0.4) (layer B.Cu) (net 23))
 (segment (start 158.75 102.99) (end 164.98 102.99) (width 0.4) (layer F.Cu) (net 6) (status 400000))
 (segment (start 164.98 102.99) (end 170.18 97.79) (width 0.4) (layer F.Cu) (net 6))
 (segment (start 170.18 97.79) (end 170.18 96.52) (width 0.4) (layer F.Cu) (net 6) (status 800000))
 (segment (start 187.96 81.28) (end 187.96 96.52) (width 0.25) (layer B.Cu) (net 6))
 (segment (start 170.18 81.28) (end 170.18 79.756) (width 0.25) (layer B.Cu) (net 6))
 (segment (start 186.69 78.994) (end 187.96 80.264) (width 0.25) (layer B.Cu) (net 6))
 (segment (start 170.942 78.994) (end 186.69 78.994) (width 0.25) (layer B.Cu) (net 6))
 (segment (start 170.18 79.756) (end 170.942 78.994) (width 0.25) (layer B.Cu) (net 6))
 (segment (start 187.96 80.264) (end 187.96 81.28) (width 0.25) (layer B.Cu) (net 6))
 (segment (start 170.18 96.52) (end 170.18 81.28) (width 0.25) (layer B.Cu) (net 6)))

